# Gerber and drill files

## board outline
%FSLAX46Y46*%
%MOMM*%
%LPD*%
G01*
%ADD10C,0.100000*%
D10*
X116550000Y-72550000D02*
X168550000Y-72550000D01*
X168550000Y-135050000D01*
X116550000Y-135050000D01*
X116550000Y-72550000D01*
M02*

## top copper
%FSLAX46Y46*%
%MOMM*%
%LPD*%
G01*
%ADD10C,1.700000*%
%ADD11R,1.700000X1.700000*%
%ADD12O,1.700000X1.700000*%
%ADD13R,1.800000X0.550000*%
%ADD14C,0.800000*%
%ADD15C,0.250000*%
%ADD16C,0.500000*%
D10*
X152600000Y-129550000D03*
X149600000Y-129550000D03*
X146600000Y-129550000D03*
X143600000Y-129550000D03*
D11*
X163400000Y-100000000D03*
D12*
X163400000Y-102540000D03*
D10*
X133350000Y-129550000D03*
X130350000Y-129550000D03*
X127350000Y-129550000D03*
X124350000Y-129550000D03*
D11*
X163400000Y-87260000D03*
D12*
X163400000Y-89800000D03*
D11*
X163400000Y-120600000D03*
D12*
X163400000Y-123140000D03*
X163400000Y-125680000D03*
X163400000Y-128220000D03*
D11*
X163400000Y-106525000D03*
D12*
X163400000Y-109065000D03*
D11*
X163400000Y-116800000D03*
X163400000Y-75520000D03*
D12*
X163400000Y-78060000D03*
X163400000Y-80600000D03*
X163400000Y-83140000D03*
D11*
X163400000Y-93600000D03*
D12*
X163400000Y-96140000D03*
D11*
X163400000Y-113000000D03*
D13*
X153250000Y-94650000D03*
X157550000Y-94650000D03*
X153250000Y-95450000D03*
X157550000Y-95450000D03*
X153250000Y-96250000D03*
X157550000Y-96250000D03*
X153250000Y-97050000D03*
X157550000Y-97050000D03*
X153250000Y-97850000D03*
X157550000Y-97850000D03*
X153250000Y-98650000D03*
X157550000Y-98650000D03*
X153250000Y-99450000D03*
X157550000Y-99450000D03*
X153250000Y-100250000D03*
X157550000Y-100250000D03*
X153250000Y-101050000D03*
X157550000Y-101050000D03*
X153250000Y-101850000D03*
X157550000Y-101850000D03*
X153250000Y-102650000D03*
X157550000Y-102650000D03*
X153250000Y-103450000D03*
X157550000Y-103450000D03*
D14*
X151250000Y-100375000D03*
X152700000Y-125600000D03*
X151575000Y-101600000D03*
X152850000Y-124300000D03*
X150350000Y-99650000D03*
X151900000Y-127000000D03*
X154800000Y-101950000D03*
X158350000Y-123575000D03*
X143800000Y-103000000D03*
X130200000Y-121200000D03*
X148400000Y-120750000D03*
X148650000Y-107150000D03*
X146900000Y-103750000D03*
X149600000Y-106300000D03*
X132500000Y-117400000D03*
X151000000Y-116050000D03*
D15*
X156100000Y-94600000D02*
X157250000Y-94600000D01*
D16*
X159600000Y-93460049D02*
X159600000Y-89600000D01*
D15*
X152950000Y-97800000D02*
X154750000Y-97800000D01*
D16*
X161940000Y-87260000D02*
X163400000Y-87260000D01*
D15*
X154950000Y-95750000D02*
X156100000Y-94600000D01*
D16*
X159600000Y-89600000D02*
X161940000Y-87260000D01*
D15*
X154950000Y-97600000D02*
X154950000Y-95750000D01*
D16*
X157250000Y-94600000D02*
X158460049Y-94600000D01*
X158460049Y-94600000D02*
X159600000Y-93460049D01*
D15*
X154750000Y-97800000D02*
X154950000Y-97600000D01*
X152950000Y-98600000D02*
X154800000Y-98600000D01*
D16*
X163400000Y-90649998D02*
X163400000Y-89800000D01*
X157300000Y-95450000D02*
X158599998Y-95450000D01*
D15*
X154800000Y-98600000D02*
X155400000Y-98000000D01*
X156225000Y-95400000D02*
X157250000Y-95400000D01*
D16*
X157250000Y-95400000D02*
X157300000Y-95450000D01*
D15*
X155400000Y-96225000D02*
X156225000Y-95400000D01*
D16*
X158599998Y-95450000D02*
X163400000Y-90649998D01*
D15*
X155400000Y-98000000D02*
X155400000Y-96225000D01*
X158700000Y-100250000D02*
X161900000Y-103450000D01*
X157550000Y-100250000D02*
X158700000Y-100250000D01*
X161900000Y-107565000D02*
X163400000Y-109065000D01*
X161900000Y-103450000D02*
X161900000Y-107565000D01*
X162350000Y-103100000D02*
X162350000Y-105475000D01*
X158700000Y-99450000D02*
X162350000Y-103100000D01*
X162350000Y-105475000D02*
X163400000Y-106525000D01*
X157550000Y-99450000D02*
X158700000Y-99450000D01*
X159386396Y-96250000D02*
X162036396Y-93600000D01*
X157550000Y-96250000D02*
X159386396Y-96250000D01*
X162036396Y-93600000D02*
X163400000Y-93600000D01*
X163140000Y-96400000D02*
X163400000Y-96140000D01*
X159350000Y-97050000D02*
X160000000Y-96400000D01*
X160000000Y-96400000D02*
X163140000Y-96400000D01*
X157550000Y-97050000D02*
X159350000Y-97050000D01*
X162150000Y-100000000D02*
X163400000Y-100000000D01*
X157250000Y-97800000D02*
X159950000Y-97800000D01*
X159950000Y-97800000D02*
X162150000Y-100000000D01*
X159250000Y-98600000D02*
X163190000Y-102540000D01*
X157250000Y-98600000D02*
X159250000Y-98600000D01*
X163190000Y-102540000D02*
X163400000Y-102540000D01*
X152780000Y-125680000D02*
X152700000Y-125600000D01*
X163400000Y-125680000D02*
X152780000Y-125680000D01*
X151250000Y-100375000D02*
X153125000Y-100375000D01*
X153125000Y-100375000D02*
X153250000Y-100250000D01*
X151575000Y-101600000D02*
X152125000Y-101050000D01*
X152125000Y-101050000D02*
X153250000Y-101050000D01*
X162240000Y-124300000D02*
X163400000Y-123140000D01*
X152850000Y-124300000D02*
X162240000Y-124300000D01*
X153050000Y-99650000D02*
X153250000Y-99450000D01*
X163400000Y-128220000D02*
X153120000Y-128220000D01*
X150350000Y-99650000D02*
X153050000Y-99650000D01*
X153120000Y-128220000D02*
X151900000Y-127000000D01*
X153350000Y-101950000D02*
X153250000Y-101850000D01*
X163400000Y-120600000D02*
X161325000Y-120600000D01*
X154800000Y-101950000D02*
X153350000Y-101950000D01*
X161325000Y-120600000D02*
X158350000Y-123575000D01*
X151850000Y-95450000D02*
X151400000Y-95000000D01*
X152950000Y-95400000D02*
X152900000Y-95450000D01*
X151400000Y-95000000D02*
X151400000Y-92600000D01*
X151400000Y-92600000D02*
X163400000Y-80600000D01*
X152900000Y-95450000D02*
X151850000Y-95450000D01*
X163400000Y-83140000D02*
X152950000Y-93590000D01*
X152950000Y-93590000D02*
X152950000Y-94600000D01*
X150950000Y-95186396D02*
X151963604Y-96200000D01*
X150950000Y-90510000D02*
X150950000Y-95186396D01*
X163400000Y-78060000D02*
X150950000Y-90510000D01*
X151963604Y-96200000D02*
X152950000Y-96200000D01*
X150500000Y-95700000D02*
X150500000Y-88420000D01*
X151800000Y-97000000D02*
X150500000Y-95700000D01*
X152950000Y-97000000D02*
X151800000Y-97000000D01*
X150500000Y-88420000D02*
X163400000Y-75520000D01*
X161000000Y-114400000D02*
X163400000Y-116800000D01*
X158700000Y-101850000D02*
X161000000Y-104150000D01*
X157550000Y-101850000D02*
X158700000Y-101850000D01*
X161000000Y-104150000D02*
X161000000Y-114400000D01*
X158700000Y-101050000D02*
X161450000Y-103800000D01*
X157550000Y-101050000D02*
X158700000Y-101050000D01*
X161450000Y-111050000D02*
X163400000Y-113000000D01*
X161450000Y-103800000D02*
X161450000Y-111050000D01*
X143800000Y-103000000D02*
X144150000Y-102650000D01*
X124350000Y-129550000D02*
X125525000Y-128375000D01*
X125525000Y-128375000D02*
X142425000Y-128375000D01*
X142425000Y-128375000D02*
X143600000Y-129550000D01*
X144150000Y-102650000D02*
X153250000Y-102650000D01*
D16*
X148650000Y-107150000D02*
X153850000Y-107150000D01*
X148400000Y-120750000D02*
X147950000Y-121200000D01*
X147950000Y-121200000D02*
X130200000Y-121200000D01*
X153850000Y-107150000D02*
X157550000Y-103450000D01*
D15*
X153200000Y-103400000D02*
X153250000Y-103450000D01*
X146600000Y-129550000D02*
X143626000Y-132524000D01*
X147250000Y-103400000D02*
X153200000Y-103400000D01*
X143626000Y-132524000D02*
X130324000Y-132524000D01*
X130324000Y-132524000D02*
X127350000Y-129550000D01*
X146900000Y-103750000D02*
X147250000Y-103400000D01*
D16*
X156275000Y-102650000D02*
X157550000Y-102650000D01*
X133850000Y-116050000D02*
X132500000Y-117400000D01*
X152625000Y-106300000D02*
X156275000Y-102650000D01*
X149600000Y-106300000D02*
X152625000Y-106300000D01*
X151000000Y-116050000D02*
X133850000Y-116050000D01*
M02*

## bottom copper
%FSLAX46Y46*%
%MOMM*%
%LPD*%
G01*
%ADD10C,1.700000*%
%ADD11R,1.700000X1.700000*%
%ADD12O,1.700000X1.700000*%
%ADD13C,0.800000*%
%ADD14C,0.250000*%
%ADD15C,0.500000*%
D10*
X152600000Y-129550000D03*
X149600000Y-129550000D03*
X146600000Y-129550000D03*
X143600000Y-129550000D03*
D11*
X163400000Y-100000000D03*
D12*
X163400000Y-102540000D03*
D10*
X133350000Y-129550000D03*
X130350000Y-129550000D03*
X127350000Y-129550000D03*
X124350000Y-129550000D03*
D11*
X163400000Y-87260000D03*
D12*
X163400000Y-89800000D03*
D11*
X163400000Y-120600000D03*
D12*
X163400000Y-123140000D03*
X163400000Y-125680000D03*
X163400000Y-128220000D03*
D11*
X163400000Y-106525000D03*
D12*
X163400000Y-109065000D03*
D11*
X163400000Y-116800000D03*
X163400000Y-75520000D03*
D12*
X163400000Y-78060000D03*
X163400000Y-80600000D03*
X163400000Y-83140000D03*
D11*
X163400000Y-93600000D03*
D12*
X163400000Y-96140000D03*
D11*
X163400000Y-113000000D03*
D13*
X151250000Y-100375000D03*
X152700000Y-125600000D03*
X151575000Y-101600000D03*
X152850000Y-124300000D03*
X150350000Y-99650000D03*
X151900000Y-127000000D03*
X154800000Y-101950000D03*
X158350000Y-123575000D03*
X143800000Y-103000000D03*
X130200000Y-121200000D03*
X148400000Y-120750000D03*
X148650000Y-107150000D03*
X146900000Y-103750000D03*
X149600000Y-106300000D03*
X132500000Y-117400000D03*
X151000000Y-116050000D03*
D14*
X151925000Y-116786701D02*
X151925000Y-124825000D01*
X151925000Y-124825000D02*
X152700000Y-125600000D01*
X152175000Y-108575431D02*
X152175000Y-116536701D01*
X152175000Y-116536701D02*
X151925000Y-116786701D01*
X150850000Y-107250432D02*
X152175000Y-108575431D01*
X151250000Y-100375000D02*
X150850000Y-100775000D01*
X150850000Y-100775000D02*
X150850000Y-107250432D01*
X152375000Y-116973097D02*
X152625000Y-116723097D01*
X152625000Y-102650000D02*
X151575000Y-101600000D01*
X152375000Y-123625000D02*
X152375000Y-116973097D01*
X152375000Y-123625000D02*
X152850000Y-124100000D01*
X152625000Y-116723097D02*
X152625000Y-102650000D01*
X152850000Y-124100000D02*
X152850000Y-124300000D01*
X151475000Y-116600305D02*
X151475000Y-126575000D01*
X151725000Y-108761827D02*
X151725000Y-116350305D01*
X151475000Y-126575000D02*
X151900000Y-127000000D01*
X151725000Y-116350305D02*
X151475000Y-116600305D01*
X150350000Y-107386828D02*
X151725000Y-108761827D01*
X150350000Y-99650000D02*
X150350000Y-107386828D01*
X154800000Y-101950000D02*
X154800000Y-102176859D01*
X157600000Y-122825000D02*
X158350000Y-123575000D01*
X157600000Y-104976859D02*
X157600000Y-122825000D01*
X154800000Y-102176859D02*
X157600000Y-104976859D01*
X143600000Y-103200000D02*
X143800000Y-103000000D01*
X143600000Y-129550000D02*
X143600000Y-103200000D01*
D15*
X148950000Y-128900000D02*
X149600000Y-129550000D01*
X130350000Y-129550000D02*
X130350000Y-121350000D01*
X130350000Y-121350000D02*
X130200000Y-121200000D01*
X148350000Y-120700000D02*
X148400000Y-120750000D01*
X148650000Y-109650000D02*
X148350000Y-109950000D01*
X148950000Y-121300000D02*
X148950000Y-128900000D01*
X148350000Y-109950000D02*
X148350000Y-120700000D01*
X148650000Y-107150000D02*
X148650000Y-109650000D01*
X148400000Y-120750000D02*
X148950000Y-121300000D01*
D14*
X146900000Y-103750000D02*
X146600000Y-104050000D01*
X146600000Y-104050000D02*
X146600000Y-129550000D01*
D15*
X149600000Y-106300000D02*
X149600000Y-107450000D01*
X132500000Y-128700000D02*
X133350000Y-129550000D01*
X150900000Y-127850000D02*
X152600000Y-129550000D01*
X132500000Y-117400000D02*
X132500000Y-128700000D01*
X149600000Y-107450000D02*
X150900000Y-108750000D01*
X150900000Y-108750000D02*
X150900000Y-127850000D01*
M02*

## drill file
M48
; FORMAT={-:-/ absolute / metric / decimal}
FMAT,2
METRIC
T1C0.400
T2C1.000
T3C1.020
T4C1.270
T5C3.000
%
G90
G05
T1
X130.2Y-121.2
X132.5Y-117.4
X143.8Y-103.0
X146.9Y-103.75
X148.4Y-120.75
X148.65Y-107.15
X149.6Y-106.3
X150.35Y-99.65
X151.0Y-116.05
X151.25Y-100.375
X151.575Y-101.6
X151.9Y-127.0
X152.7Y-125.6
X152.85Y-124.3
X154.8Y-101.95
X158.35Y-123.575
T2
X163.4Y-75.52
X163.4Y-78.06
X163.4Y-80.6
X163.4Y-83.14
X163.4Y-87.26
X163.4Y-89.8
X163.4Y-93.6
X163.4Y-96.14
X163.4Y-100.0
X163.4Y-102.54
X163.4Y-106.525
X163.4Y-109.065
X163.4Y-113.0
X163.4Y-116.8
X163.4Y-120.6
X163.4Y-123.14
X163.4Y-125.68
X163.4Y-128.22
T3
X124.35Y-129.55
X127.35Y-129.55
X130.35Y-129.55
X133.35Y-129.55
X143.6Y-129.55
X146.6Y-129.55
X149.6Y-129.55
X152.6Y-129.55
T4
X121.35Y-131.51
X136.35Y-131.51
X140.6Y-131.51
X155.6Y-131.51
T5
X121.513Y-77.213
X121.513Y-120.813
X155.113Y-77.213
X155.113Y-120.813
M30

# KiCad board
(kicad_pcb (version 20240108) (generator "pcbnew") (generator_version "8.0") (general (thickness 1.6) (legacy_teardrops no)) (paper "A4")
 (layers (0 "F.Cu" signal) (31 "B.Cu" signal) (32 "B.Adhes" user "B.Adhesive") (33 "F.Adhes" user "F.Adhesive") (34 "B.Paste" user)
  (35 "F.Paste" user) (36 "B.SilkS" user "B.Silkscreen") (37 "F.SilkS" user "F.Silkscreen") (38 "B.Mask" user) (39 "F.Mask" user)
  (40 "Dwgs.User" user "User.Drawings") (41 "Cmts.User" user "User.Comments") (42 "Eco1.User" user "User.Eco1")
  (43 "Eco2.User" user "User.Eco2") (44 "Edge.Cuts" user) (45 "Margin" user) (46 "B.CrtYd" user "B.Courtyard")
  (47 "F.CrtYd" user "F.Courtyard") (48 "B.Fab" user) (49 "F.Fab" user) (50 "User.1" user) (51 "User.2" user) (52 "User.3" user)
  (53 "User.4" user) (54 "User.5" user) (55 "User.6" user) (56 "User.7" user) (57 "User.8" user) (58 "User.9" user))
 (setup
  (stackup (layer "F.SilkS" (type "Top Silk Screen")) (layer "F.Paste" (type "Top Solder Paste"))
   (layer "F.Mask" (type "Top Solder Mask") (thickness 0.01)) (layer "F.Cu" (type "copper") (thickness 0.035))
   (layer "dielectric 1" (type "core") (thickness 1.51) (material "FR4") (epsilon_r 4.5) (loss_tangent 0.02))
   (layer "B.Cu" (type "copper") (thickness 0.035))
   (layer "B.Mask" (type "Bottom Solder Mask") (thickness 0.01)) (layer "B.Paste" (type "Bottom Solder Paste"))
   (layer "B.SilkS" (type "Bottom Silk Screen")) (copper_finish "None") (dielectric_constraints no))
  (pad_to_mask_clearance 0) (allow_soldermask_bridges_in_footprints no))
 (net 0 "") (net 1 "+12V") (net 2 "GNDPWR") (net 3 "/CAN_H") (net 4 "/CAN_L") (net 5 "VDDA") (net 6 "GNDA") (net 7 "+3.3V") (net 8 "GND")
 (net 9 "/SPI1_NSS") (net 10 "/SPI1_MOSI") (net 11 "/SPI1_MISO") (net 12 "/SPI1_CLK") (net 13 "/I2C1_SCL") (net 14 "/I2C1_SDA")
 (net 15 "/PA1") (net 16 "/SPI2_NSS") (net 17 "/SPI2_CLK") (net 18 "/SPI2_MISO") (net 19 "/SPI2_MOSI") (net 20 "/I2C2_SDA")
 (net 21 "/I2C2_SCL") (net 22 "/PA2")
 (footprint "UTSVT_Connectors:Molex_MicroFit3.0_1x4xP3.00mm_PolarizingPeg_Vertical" (layer "F.Cu") (at 152.6 129.55 180)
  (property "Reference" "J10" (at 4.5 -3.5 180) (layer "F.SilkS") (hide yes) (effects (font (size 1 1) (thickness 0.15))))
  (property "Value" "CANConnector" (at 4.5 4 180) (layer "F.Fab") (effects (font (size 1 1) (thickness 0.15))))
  (pad "" np_thru_hole circle (at -3 -1.96 180) (size 1.27 1.27) (drill 1.27) (layers "*.Cu" "*.Mask"))
  (pad "" np_thru_hole circle (at 12 -1.96 180) (size 1.27 1.27) (drill 1.27) (layers "*.Cu" "*.Mask"))
  (pad "1" thru_hole circle (at 0 0 180) (size 1.7 1.7) (drill 1.02) (layers "*.Cu" "*.Mask") (remove_unused_layers no) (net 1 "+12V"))
  (pad "2" thru_hole circle (at 3 0 180) (size 1.7 1.7) (drill 1.02) (layers "*.Cu" "*.Mask") (remove_unused_layers no) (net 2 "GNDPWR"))
  (pad "3" thru_hole circle (at 6 0 180) (size 1.7 1.7) (drill 1.02) (layers "*.Cu" "*.Mask") (remove_unused_layers no) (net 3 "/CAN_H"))
  (pad "4" thru_hole circle (at 9 0 180) (size 1.7 1.7) (drill 1.02) (layers "*.Cu" "*.Mask") (remove_unused_layers no) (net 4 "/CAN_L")))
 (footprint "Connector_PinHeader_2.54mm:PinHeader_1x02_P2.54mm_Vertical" (layer "F.Cu") (at 163.4 100)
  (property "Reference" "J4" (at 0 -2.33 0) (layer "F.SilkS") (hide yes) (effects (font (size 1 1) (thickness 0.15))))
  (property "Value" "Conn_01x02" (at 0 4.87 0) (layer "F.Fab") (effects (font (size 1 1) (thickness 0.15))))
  (pad "1" thru_hole rect (at 0 0) (size 1.7 1.7) (drill 1) (layers "*.Cu" "*.Mask") (remove_unused_layers no) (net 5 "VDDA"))
  (pad "2" thru_hole oval (at 0 2.54) (size 1.7 1.7) (drill 1) (layers "*.Cu" "*.Mask") (remove_unused_layers no) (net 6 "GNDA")))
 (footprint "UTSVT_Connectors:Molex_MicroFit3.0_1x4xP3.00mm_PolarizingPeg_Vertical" (layer "F.Cu") (at 133.35 129.55 180)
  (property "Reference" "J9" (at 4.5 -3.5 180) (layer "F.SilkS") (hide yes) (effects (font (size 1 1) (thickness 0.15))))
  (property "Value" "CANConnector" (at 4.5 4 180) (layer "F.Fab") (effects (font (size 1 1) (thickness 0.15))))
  (pad "" np_thru_hole circle (at -3 -1.96 180) (size 1.27 1.27) (drill 1.27) (layers "*.Cu" "*.Mask"))
  (pad "" np_thru_hole circle (at 12 -1.96 180) (size 1.27 1.27) (drill 1.27) (layers "*.Cu" "*.Mask"))
  (pad "1" thru_hole circle (at 0 0 180) (size 1.7 1.7) (drill 1.02) (layers "*.Cu" "*.Mask") (remove_unused_layers no) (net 1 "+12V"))
  (pad "2" thru_hole circle (at 3 0 180) (size 1.7 1.7) (drill 1.02) (layers "*.Cu" "*.Mask") (remove_unused_layers no) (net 2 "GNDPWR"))
  (pad "3" thru_hole circle (at 6 0 180) (size 1.7 1.7) (drill 1.02) (layers "*.Cu" "*.Mask") (remove_unused_layers no) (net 3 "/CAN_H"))
  (pad "4" thru_hole circle (at 9 0 180) (size 1.7 1.7) (drill 1.02) (layers "*.Cu" "*.Mask") (remove_unused_layers no) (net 4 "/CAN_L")))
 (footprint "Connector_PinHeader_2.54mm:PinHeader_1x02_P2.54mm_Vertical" (layer "F.Cu") (at 163.4 87.26)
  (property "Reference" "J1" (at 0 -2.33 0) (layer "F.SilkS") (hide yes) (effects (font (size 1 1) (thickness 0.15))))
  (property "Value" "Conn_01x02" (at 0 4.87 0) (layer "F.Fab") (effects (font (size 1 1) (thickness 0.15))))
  (pad "1" thru_hole rect (at 0 0) (size 1.7 1.7) (drill 1) (layers "*.Cu" "*.Mask") (remove_unused_layers no) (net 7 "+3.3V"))
  (pad "2" thru_hole oval (at 0 2.54) (size 1.7 1.7) (drill 1) (layers "*.Cu" "*.Mask") (remove_unused_layers no) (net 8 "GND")))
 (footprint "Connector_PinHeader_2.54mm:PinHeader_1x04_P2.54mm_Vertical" (layer "F.Cu") (at 163.4 120.6)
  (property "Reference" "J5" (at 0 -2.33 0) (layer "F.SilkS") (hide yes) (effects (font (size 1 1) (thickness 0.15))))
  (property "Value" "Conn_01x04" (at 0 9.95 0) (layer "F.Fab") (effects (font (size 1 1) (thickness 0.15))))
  (pad "1" thru_hole rect (at 0 0) (size 1.7 1.7) (drill 1) (layers "*.Cu" "*.Mask") (remove_unused_layers no) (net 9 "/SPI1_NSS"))
  (pad "2" thru_hole oval (at 0 2.54) (size 1.7 1.7) (drill 1) (layers "*.Cu" "*.Mask") (remove_unused_layers no) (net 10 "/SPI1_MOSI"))
  (pad "3" thru_hole oval (at 0 5.08) (size 1.7 1.7) (drill 1) (layers "*.Cu" "*.Mask") (remove_unused_layers no) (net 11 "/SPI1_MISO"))
  (pad "4" thru_hole oval (at 0 7.62) (size 1.7 1.7) (drill 1) (layers "*.Cu" "*.Mask") (remove_unused_layers no) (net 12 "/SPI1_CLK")))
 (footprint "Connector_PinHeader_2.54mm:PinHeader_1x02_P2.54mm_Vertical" (layer "F.Cu") (at 163.4 106.525)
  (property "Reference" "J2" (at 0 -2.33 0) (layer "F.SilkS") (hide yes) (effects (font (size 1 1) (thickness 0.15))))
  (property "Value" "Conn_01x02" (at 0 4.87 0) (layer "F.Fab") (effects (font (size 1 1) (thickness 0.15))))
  (pad "1" thru_hole rect (at 0 0) (size 1.7 1.7) (drill 1) (layers "*.Cu" "*.Mask") (remove_unused_layers no) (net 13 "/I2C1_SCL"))
  (pad "2" thru_hole oval (at 0 2.54) (size 1.7 1.7) (drill 1) (layers "*.Cu" "*.Mask") (remove_unused_layers no) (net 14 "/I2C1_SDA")))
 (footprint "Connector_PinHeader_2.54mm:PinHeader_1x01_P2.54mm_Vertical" (layer "F.Cu") (at 163.4 116.8)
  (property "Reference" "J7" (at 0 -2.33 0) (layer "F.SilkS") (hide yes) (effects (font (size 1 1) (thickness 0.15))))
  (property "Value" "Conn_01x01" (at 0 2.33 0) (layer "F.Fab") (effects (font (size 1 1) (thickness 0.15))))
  (pad "1" thru_hole rect (at 0 0) (size 1.7 1.7) (drill 1) (layers "*.Cu" "*.Mask") (remove_unused_layers no) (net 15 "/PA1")))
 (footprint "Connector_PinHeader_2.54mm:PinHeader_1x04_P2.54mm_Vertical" (layer "F.Cu") (at 163.4 75.52)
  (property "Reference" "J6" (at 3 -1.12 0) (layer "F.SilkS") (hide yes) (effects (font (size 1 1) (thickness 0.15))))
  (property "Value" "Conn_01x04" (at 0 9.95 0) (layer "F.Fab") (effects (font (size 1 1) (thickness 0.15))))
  (pad "1" thru_hole rect (at 0 0) (size 1.7 1.7) (drill 1) (layers "*.Cu" "*.Mask") (remove_unused_layers no) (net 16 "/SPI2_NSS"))
  (pad "2" thru_hole oval (at 0 2.54) (size 1.7 1.7) (drill 1) (layers "*.Cu" "*.Mask") (remove_unused_layers no) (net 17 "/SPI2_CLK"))
  (pad "3" thru_hole oval (at 0 5.08) (size 1.7 1.7) (drill 1) (layers "*.Cu" "*.Mask") (remove_unused_layers no) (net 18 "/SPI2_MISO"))
  (pad "4" thru_hole oval (at 0 7.62) (size 1.7 1.7) (drill 1) (layers "*.Cu" "*.Mask") (remove_unused_layers no) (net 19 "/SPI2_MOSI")))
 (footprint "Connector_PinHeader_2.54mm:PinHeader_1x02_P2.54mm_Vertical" (layer "F.Cu") (at 163.4 93.6)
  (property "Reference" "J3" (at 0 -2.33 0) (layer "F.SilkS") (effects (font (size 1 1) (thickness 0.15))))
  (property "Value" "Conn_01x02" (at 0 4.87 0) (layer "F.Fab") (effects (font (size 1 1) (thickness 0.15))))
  (pad "1" thru_hole rect (at 0 0) (size 1.7 1.7) (drill 1) (layers "*.Cu" "*.Mask") (remove_unused_layers no) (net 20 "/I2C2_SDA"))
  (pad "2" thru_hole oval (at 0 2.54) (size 1.7 1.7) (drill 1) (layers "*.Cu" "*.Mask") (remove_unused_layers no) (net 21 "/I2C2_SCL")))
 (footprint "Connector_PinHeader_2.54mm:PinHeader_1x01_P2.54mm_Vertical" (layer "F.Cu") (at 163.4 113)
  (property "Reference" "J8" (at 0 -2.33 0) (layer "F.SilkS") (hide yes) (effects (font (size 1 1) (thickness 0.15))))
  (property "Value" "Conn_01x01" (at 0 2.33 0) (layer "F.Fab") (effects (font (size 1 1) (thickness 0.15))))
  (pad "1" thru_hole rect (at 0 0) (size 1.7 1.7) (drill 1) (layers "*.Cu" "*.Mask") (remove_unused_layers no) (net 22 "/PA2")))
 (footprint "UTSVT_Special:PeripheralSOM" (layer "F.Cu") (at 137.075 95.825)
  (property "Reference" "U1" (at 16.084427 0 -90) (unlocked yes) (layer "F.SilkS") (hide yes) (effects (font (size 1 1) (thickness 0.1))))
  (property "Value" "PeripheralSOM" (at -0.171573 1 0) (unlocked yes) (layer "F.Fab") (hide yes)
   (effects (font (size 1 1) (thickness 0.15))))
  (pad "" np_thru_hole circle (at -15.56226 -18.61226) (size 3 3) (drill 3) (layers "*.Cu" "*.Mask"))
  (pad "" np_thru_hole circle (at -15.56226 24.98774) (size 3 3) (drill 3) (layers "*.Cu" "*.Mask"))
  (pad "" np_thru_hole circle (at 18.03774 -18.61226) (size 3 3) (drill 3) (layers "*.Cu" "*.Mask"))
  (pad "" np_thru_hole circle (at 18.03774 24.98774) (size 3 3) (drill 3) (layers "*.Cu" "*.Mask"))
  (pad "1" smd rect (at 16.175 -1.175 90) (size 0.55 1.8) (layers "F.Cu" "F.Paste" "F.Mask") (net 19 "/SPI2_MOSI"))
  (pad "2" smd rect (at 20.475 -1.175 90) (size 0.55 1.8) (layers "F.Cu" "F.Paste" "F.Mask") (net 7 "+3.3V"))
  (pad "3" smd rect (at 16.175 -0.375 90) (size 0.55 1.8) (layers "F.Cu" "F.Paste" "F.Mask") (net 18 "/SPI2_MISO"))
  (pad "4" smd rect (at 20.475 -0.375 90) (size 0.55 1.8) (layers "F.Cu" "F.Paste" "F.Mask") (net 8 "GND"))
  (pad "5" smd rect (at 16.175 0.425 90) (size 0.55 1.8) (layers "F.Cu" "F.Paste" "F.Mask") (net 17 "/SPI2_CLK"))
  (pad "6" smd rect (at 20.475 0.425 90) (size 0.55 1.8) (layers "F.Cu" "F.Paste" "F.Mask") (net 20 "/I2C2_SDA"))
  (pad "7" smd rect (at 16.175 1.225 90) (size 0.55 1.8) (layers "F.Cu" "F.Paste" "F.Mask") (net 16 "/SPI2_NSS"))
  (pad "8" smd rect (at 20.475 1.225 90) (size 0.55 1.8) (layers "F.Cu" "F.Paste" "F.Mask") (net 21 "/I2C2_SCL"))
  (pad "9" smd rect (at 16.175 2.025 90) (size 0.55 1.8) (layers "F.Cu" "F.Paste" "F.Mask") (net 7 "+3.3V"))
  (pad "10" smd rect (at 20.475 2.025 90) (size 0.55 1.8) (layers "F.Cu" "F.Paste" "F.Mask") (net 5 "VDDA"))
  (pad "11" smd rect (at 16.175 2.825 90) (size 0.55 1.8) (layers "F.Cu" "F.Paste" "F.Mask") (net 8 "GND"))
  (pad "12" smd rect (at 20.475 2.825 90) (size 0.55 1.8) (layers "F.Cu" "F.Paste" "F.Mask") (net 6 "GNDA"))
  (pad "13" smd rect (at 16.175 3.625 90) (size 0.55 1.8) (layers "F.Cu" "F.Paste" "F.Mask") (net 12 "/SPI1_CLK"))
  (pad "14" smd rect (at 20.475 3.625 90) (size 0.55 1.8) (layers "F.Cu" "F.Paste" "F.Mask") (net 13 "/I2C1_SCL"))
  (pad "15" smd rect (at 16.175 4.425 90) (size 0.55 1.8) (layers "F.Cu" "F.Paste" "F.Mask") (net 11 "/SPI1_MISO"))
  (pad "16" smd rect (at 20.475 4.425 90) (size 0.55 1.8) (layers "F.Cu" "F.Paste" "F.Mask") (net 14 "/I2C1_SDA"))
  (pad "17" smd rect (at 16.175 5.225 90) (size 0.55 1.8) (layers "F.Cu" "F.Paste" "F.Mask") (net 10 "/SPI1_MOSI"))
  (pad "18" smd rect (at 20.475 5.225 90) (size 0.55 1.8) (layers "F.Cu" "F.Paste" "F.Mask") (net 22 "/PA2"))
  (pad "19" smd rect (at 16.175 6.025 90) (size 0.55 1.8) (layers "F.Cu" "F.Paste" "F.Mask") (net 9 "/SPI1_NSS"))
  (pad "20" smd rect (at 20.475 6.025 90) (size 0.55 1.8) (layers "F.Cu" "F.Paste" "F.Mask") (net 15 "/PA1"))
  (pad "21" smd rect (at 16.175 6.825 90) (size 0.55 1.8) (layers "F.Cu" "F.Paste" "F.Mask") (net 4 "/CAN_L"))
  (pad "22" smd rect (at 20.475 6.825 90) (size 0.55 1.8) (layers "F.Cu" "F.Paste" "F.Mask") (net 1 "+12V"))
  (pad "23" smd rect (at 16.175 7.625 90) (size 0.55 1.8) (layers "F.Cu" "F.Paste" "F.Mask") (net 3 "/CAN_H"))
  (pad "24" smd rect (at 20.475 7.625 90) (size 0.55 1.8) (layers "F.Cu" "F.Paste" "F.Mask") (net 2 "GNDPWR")))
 (gr_rect (start 116.55 72.55) (end 168.55 135.05) (stroke (width 0.1) (type default)) (fill none) (layer "Edge.Cuts"))
 (segment (start 156.1 94.6) (end 157.25 94.6) (width 0.25) (layer "F.Cu") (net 7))
 (segment (start 159.6 93.460049) (end 159.6 89.6) (width 0.5) (layer "F.Cu") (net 7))
 (segment (start 152.95 97.8) (end 154.75 97.8) (width 0.25) (layer "F.Cu") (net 7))
 (segment (start 161.94 87.26) (end 163.4 87.26) (width 0.5) (layer "F.Cu") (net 7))
 (segment (start 154.95 95.75) (end 156.1 94.6) (width 0.25) (layer "F.Cu") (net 7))
 (segment (start 159.6 89.6) (end 161.94 87.26) (width 0.5) (layer "F.Cu") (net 7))
 (segment (start 154.95 97.6) (end 154.95 95.75) (width 0.25) (layer "F.Cu") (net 7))
 (segment (start 157.25 94.6) (end 158.460049 94.6) (width 0.5) (layer "F.Cu") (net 7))
 (segment (start 158.460049 94.6) (end 159.6 93.460049) (width 0.5) (layer "F.Cu") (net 7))
 (segment (start 154.75 97.8) (end 154.95 97.6) (width 0.25) (layer "F.Cu") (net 7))
 (segment (start 152.95 98.6) (end 154.8 98.6) (width 0.25) (layer "F.Cu") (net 8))
 (segment (start 163.4 90.649998) (end 163.4 89.8) (width 0.5) (layer "F.Cu") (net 8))
 (segment (start 157.3 95.45) (end 158.599998 95.45) (width 0.5) (layer "F.Cu") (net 8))
 (segment (start 154.8 98.6) (end 155.4 98) (width 0.25) (layer "F.Cu") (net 8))
 (segment (start 156.225 95.4) (end 157.25 95.4) (width 0.25) (layer "F.Cu") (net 8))
 (segment (start 157.25 95.4) (end 157.3 95.45) (width 0.5) (layer "F.Cu") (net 8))
 (segment (start 155.4 96.225) (end 156.225 95.4) (width 0.25) (layer "F.Cu") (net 8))
 (segment (start 158.599998 95.45) (end 163.4 90.649998) (width 0.5) (layer "F.Cu") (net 8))
 (segment (start 155.4 98) (end 155.4 96.225) (width 0.25) (layer "F.Cu") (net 8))
 (segment (start 158.7 100.25) (end 161.9 103.45) (width 0.25) (layer "F.Cu") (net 14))
 (segment (start 157.55 100.25) (end 158.7 100.25) (width 0.25) (layer "F.Cu") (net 14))
 (segment (start 161.9 107.565) (end 163.4 109.065) (width 0.25) (layer "F.Cu") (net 14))
 (segment (start 161.9 103.45) (end 161.9 107.565) (width 0.25) (layer "F.Cu") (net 14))
 (segment (start 162.35 103.1) (end 162.35 105.475) (width 0.25) (layer "F.Cu") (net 13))
 (segment (start 158.7 99.45) (end 162.35 103.1) (width 0.25) (layer "F.Cu") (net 13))
 (segment (start 162.35 105.475) (end 163.4 106.525) (width 0.25) (layer "F.Cu") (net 13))
 (segment (start 157.55 99.45) (end 158.7 99.45) (width 0.25) (layer "F.Cu") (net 13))
 (segment (start 159.386396 96.25) (end 162.036396 93.6) (width 0.25) (layer "F.Cu") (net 20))
 (segment (start 157.55 96.25) (end 159.386396 96.25) (width 0.25) (layer "F.Cu") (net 20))
 (segment (start 162.036396 93.6) (end 163.4 93.6) (width 0.25) (layer "F.Cu") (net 20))
 (segment (start 163.14 96.4) (end 163.4 96.14) (width 0.25) (layer "F.Cu") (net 21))
 (segment (start 159.35 97.05) (end 160 96.4) (width 0.25) (layer "F.Cu") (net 21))
 (segment (start 160 96.4) (end 163.14 96.4) (width 0.25) (layer "F.Cu") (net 21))
 (segment (start 157.55 97.05) (end 159.35 97.05) (width 0.25) (layer "F.Cu") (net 21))
 (segment (start 162.15 100) (end 163.4 100) (width 0.25) (layer "F.Cu") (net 5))
 (segment (start 157.25 97.8) (end 159.95 97.8) (width 0.25) (layer "F.Cu") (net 5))
 (segment (start 159.95 97.8) (end 162.15 100) (width 0.25) (layer "F.Cu") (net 5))
 (segment (start 159.25 98.6) (end 163.19 102.54) (width 0.25) (layer "F.Cu") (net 6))
 (segment (start 157.25 98.6) (end 159.25 98.6) (width 0.25) (layer "F.Cu") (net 6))
 (segment (start 163.19 102.54) (end 163.4 102.54) (width 0.25) (layer "F.Cu") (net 6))
 (segment (start 152.78 125.68) (end 152.7 125.6) (width 0.25) (layer "F.Cu") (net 11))
 (segment (start 163.4 125.68) (end 152.78 125.68) (width 0.25) (layer "F.Cu") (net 11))
 (segment (start 151.25 100.375) (end 153.125 100.375) (width 0.25) (layer "F.Cu") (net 11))
 (segment (start 153.125 100.375) (end 153.25 100.25) (width 0.25) (layer "F.Cu") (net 11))
 (via (at 151.25 100.375) (size 0.8) (drill 0.4) (layers "F.Cu" "B.Cu") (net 11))
 (via (at 152.7 125.6) (size 0.8) (drill 0.4) (layers "F.Cu" "B.Cu") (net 11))
 (segment (start 151.925 116.786701) (end 151.925 124.825) (width 0.25) (layer "B.Cu") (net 11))
 (segment (start 151.925 124.825) (end 152.7 125.6) (width 0.25) (layer "B.Cu") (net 11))
 (segment (start 152.175 108.575431) (end 152.175 116.536701) (width 0.25) (layer "B.Cu") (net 11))
 (segment (start 152.175 116.536701) (end 151.925 116.786701) (width 0.25) (layer "B.Cu") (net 11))
 (segment (start 150.85 107.250432) (end 152.175 108.575431) (width 0.25) (layer "B.Cu") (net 11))
 (segment (start 151.25 100.375) (end 150.85 100.775) (width 0.25) (layer "B.Cu") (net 11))
 (segment (start 150.85 100.775) (end 150.85 107.250432) (width 0.25) (layer "B.Cu") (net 11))
 (segment (start 151.575 101.6) (end 152.125 101.05) (width 0.25) (layer "F.Cu") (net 10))
 (segment (start 152.125 101.05) (end 153.25 101.05) (width 0.25) (layer "F.Cu") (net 10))
 (segment (start 162.24 124.3) (end 163.4 123.14) (width 0.25) (layer "F.Cu") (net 10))
 (segment (start 152.85 124.3) (end 162.24 124.3) (width 0.25) (layer "F.Cu") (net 10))
 (via (at 151.575 101.6) (size 0.8) (drill 0.4) (layers "F.Cu" "B.Cu") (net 10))
 (via (at 152.85 124.3) (size 0.8) (drill 0.4) (layers "F.Cu" "B.Cu") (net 10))
 (segment (start 152.375 116.973097) (end 152.625 116.723097) (width 0.25) (layer "B.Cu") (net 10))
 (segment (start 152.625 102.65) (end 151.575 101.6) (width 0.25) (layer "B.Cu") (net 10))
 (segment (start 152.375 123.625) (end 152.375 116.973097) (width 0.25) (layer "B.Cu") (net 10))
 (segment (start 152.375 123.625) (end 152.85 124.1) (width 0.25) (layer "B.Cu") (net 10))
 (segment (start 152.625 116.723097) (end 152.625 102.65) (width 0.25) (layer "B.Cu") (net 10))
 (segment (start 152.85 124.1) (end 152.85 124.3) (width 0.25) (layer "B.Cu") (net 10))
 (segment (start 153.05 99.65) (end 153.25 99.45) (width 0.25) (layer "F.Cu") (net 12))
 (segment (start 163.4 128.22) (end 153.12 128.22) (width 0.25) (layer "F.Cu") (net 12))
 (segment (start 150.35 99.65) (end 153.05 99.65) (width 0.25) (layer "F.Cu") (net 12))
 (segment (start 153.12 128.22) (end 151.9 127) (width 0.25) (layer "F.Cu") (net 12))
 (via (at 150.35 99.65) (size 0.8) (drill 0.4) (layers "F.Cu" "B.Cu") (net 12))
 (via (at 151.9 127) (size 0.8) (drill 0.4) (layers "F.Cu" "B.Cu") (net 12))
 (segment (start 151.475 116.600305) (end 151.475 126.575) (width 0.25) (layer "B.Cu") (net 12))
 (segment (start 151.725 108.761827) (end 151.725 116.350305) (width 0.25) (layer "B.Cu") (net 12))
 (segment (start 151.475 126.575) (end 151.9 127) (width 0.25) (layer "B.Cu") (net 12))
 (segment (start 151.725 116.350305) (end 151.475 116.600305) (width 0.25) (layer "B.Cu") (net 12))
 (segment (start 150.35 107.386828) (end 151.725 108.761827) (width 0.25) (layer "B.Cu") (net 12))
 (segment (start 150.35 99.65) (end 150.35 107.386828) (width 0.25) (layer "B.Cu") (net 12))
 (segment (start 153.35 101.95) (end 153.25 101.85) (width 0.25) (layer "F.Cu") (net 9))
 (segment (start 163.4 120.6) (end 161.325 120.6) (width 0.25) (layer "F.Cu") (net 9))
 (segment (start 154.8 101.95) (end 153.35 101.95) (width 0.25) (layer "F.Cu") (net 9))
 (segment (start 161.325 120.6) (end 158.35 123.575) (width 0.25) (layer "F.Cu") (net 9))
 (via (at 154.8 101.95) (size 0.8) (drill 0.4) (layers "F.Cu" "B.Cu") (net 9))
 (via (at 158.35 123.575) (size 0.8) (drill 0.4) (layers "F.Cu" "B.Cu") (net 9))
 (segment (start 154.8 101.95) (end 154.8 102.176859) (width 0.25) (layer "B.Cu") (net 9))
 (segment (start 157.6 122.825) (end 158.35 123.575) (width 0.25) (layer "B.Cu") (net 9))
 (segment (start 157.6 104.976859) (end 157.6 122.825) (width 0.25) (layer "B.Cu") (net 9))
 (segment (start 154.8 102.176859) (end 157.6 104.976859) (width 0.25) (layer "B.Cu") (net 9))
 (segment (start 151.85 95.45) (end 151.4 95) (width 0.25) (layer "F.Cu") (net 18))
 (segment (start 152.95 95.4) (end 152.9 95.45) (width 0.25) (layer "F.Cu") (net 18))
 (segment (start 151.4 95) (end 151.4 92.6) (width 0.25) (layer "F.Cu") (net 18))
 (segment (start 151.4 92.6) (end 163.4 80.6) (width 0.25) (layer "F.Cu") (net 18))
 (segment (start 152.9 95.45) (end 151.85 95.45) (width 0.25) (layer "F.Cu") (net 18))
 (segment (start 163.4 83.14) (end 152.95 93.59) (width 0.25) (layer "F.Cu") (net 19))
 (segment (start 152.95 93.59) (end 152.95 94.6) (width 0.25) (layer "F.Cu") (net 19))
 (segment (start 150.95 95.186396) (end 151.963604 96.2) (width 0.25) (layer "F.Cu") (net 17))
 (segment (start 150.95 90.51) (end 150.95 95.186396) (width 0.25) (layer "F.Cu") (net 17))
 (segment (start 163.4 78.06) (end 150.95 90.51) (width 0.25) (layer "F.Cu") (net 17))
 (segment (start 151.963604 96.2) (end 152.95 96.2) (width 0.25) (layer "F.Cu") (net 17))
 (segment (start 150.5 95.7) (end 150.5 88.42) (width 0.25) (layer "F.Cu") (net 16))
 (segment (start 151.8 97) (end 150.5 95.7) (width 0.25) (layer "F.Cu") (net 16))
 (segment (start 152.95 97) (end 151.8 97) (width 0.25) (layer "F.Cu") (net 16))
 (segment (start 150.5 88.42) (end 163.4 75.52) (width 0.25) (layer "F.Cu") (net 16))
 (segment (start 161 114.4) (end 163.4 116.8) (width 0.25) (layer "F.Cu") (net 15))
 (segment (start 158.7 101.85) (end 161 104.15) (width 0.25) (layer "F.Cu") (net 15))
 (segment (start 157.55 101.85) (end 158.7 101.85) (width 0.25) (layer "F.Cu") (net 15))
 (segment (start 161 104.15) (end 161 114.4) (width 0.25) (layer "F.Cu") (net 15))
 (segment (start 158.7 101.05) (end 161.45 103.8) (width 0.25) (layer "F.Cu") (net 22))
 (segment (start 157.55 101.05) (end 158.7 101.05) (width 0.25) (layer "F.Cu") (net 22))
 (segment (start 161.45 111.05) (end 163.4 113) (width 0.25) (layer "F.Cu") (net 22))
 (segment (start 161.45 103.8) (end 161.45 111.05) (width 0.25) (layer "F.Cu") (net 22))
 (segment (start 143.8 103) (end 144.15 102.65) (width 0.25) (layer "F.Cu") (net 4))
 (segment (start 124.35 129.55) (end 125.525 128.375) (width 0.25) (layer "F.Cu") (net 4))
 (segment (start 125.525 128.375) (end 142.425 128.375) (width 0.25) (layer "F.Cu") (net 4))
 (segment (start 142.425 128.375) (end 143.6 129.55) (width 0.25) (layer "F.Cu") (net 4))
 (segment (start 144.15 102.65) (end 153.25 102.65) (width 0.25) (layer "F.Cu") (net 4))
 (via (at 143.8 103) (size 0.8) (drill 0.4) (layers "F.Cu" "B.Cu") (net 4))
 (segment (start 143.6 103.2) (end 143.8 103) (width 0.25) (layer "B.Cu") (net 4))
 (segment (start 143.6 129.55) (end 143.6 103.2) (width 0.25) (layer "B.Cu") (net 4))
 (segment (start 148.65 107.15) (end 153.85 107.15) (width 0.5) (layer "F.Cu") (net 2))
 (segment (start 148.4 120.75) (end 147.95 121.2) (width 0.5) (layer "F.Cu") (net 2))
 (segment (start 147.95 121.2) (end 130.2 121.2) (width 0.5) (layer "F.Cu") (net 2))
 (segment (start 153.85 107.15) (end 157.55 103.45) (width 0.5) (layer "F.Cu") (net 2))
 (via (at 130.2 121.2) (size 0.8) (drill 0.4) (layers "F.Cu" "B.Cu") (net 2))
 (via (at 148.4 120.75) (size 0.8) (drill 0.4) (layers "F.Cu" "B.Cu") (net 2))
 (via (at 148.65 107.15) (size 0.8) (drill 0.4) (layers "F.Cu" "B.Cu") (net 2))
 (segment (start 148.95 128.9) (end 149.6 129.55) (width 0.5) (layer "B.Cu") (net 2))
 (segment (start 130.35 129.55) (end 130.35 121.35) (width 0.5) (layer "B.Cu") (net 2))
 (segment (start 130.35 121.35) (end 130.2 121.2) (width 0.5) (layer "B.Cu") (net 2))
 (segment (start 148.35 120.7) (end 148.4 120.75) (width 0.5) (layer "B.Cu") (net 2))
 (segment (start 148.65 109.65) (end 148.35 109.95) (width 0.5) (layer "B.Cu") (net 2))
 (segment (start 148.95 121.3) (end 148.95 128.9) (width 0.5) (layer "B.Cu") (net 2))
 (segment (start 148.35 109.95) (end 148.35 120.7) (width 0.5) (layer "B.Cu") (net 2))
 (segment (start 148.65 107.15) (end 148.65 109.65) (width 0.5) (layer "B.Cu") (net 2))
 (segment (start 148.4 120.75) (end 148.95 121.3) (width 0.5) (layer "B.Cu") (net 2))
 (segment (start 153.2 103.4) (end 153.25 103.45) (width 0.25) (layer "F.Cu") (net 3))
 (segment (start 146.6 129.55) (end 143.626 132.524) (width 0.25) (layer "F.Cu") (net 3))
 (segment (start 147.25 103.4) (end 153.2 103.4) (width 0.25) (layer "F.Cu") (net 3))
 (segment (start 143.626 132.524) (end 130.324 132.524) (width 0.25) (layer "F.Cu") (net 3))
 (segment (start 130.324 132.524) (end 127.35 129.55) (width 0.25) (layer "F.Cu") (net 3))
 (segment (start 146.9 103.75) (end 147.25 103.4) (width 0.25) (layer "F.Cu") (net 3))
 (via (at 146.9 103.75) (size 0.8) (drill 0.4) (layers "F.Cu" "B.Cu") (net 3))
 (segment (start 146.9 103.75) (end 146.6 104.05) (width 0.25) (layer "B.Cu") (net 3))
 (segment (start 146.6 104.05) (end 146.6 129.55) (width 0.25) (layer "B.Cu") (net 3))
 (segment (start 156.275 102.65) (end 157.55 102.65) (width 0.5) (layer "F.Cu") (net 1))
 (segment (start 133.85 116.05) (end 132.5 117.4) (width 0.5) (layer "F.Cu") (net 1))
 (segment (start 152.625 106.3) (end 156.275 102.65) (width 0.5) (layer "F.Cu") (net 1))
 (segment (start 149.6 106.3) (end 152.625 106.3) (width 0.5) (layer "F.Cu") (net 1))
 (segment (start 151 116.05) (end 133.85 116.05) (width 0.5) (layer "F.Cu") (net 1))
 (via (at 149.6 106.3) (size 0.8) (drill 0.4) (layers "F.Cu" "B.Cu") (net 1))
 (via (at 132.5 117.4) (size 0.8) (drill 0.4) (layers "F.Cu" "B.Cu") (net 1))
 (via (at 151 116.05) (size 0.8) (drill 0.4) (layers "F.Cu" "B.Cu") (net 1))
 (segment (start 149.6 106.3) (end 149.6 107.45) (width 0.5) (layer "B.Cu") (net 1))
 (segment (start 132.5 128.7) (end 133.35 129.55) (width 0.5) (layer "B.Cu") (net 1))
 (segment (start 150.9 127.85) (end 152.6 129.55) (width 0.5) (layer "B.Cu") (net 1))
 (segment (start 132.5 117.4) (end 132.5 128.7) (width 0.5) (layer "B.Cu") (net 1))
 (segment (start 149.6 107.45) (end 150.9 108.75) (width 0.5) (layer "B.Cu") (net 1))
 (segment (start 150.9 108.75) (end 150.9 127.85) (width 0.5) (layer "B.Cu") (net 1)))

